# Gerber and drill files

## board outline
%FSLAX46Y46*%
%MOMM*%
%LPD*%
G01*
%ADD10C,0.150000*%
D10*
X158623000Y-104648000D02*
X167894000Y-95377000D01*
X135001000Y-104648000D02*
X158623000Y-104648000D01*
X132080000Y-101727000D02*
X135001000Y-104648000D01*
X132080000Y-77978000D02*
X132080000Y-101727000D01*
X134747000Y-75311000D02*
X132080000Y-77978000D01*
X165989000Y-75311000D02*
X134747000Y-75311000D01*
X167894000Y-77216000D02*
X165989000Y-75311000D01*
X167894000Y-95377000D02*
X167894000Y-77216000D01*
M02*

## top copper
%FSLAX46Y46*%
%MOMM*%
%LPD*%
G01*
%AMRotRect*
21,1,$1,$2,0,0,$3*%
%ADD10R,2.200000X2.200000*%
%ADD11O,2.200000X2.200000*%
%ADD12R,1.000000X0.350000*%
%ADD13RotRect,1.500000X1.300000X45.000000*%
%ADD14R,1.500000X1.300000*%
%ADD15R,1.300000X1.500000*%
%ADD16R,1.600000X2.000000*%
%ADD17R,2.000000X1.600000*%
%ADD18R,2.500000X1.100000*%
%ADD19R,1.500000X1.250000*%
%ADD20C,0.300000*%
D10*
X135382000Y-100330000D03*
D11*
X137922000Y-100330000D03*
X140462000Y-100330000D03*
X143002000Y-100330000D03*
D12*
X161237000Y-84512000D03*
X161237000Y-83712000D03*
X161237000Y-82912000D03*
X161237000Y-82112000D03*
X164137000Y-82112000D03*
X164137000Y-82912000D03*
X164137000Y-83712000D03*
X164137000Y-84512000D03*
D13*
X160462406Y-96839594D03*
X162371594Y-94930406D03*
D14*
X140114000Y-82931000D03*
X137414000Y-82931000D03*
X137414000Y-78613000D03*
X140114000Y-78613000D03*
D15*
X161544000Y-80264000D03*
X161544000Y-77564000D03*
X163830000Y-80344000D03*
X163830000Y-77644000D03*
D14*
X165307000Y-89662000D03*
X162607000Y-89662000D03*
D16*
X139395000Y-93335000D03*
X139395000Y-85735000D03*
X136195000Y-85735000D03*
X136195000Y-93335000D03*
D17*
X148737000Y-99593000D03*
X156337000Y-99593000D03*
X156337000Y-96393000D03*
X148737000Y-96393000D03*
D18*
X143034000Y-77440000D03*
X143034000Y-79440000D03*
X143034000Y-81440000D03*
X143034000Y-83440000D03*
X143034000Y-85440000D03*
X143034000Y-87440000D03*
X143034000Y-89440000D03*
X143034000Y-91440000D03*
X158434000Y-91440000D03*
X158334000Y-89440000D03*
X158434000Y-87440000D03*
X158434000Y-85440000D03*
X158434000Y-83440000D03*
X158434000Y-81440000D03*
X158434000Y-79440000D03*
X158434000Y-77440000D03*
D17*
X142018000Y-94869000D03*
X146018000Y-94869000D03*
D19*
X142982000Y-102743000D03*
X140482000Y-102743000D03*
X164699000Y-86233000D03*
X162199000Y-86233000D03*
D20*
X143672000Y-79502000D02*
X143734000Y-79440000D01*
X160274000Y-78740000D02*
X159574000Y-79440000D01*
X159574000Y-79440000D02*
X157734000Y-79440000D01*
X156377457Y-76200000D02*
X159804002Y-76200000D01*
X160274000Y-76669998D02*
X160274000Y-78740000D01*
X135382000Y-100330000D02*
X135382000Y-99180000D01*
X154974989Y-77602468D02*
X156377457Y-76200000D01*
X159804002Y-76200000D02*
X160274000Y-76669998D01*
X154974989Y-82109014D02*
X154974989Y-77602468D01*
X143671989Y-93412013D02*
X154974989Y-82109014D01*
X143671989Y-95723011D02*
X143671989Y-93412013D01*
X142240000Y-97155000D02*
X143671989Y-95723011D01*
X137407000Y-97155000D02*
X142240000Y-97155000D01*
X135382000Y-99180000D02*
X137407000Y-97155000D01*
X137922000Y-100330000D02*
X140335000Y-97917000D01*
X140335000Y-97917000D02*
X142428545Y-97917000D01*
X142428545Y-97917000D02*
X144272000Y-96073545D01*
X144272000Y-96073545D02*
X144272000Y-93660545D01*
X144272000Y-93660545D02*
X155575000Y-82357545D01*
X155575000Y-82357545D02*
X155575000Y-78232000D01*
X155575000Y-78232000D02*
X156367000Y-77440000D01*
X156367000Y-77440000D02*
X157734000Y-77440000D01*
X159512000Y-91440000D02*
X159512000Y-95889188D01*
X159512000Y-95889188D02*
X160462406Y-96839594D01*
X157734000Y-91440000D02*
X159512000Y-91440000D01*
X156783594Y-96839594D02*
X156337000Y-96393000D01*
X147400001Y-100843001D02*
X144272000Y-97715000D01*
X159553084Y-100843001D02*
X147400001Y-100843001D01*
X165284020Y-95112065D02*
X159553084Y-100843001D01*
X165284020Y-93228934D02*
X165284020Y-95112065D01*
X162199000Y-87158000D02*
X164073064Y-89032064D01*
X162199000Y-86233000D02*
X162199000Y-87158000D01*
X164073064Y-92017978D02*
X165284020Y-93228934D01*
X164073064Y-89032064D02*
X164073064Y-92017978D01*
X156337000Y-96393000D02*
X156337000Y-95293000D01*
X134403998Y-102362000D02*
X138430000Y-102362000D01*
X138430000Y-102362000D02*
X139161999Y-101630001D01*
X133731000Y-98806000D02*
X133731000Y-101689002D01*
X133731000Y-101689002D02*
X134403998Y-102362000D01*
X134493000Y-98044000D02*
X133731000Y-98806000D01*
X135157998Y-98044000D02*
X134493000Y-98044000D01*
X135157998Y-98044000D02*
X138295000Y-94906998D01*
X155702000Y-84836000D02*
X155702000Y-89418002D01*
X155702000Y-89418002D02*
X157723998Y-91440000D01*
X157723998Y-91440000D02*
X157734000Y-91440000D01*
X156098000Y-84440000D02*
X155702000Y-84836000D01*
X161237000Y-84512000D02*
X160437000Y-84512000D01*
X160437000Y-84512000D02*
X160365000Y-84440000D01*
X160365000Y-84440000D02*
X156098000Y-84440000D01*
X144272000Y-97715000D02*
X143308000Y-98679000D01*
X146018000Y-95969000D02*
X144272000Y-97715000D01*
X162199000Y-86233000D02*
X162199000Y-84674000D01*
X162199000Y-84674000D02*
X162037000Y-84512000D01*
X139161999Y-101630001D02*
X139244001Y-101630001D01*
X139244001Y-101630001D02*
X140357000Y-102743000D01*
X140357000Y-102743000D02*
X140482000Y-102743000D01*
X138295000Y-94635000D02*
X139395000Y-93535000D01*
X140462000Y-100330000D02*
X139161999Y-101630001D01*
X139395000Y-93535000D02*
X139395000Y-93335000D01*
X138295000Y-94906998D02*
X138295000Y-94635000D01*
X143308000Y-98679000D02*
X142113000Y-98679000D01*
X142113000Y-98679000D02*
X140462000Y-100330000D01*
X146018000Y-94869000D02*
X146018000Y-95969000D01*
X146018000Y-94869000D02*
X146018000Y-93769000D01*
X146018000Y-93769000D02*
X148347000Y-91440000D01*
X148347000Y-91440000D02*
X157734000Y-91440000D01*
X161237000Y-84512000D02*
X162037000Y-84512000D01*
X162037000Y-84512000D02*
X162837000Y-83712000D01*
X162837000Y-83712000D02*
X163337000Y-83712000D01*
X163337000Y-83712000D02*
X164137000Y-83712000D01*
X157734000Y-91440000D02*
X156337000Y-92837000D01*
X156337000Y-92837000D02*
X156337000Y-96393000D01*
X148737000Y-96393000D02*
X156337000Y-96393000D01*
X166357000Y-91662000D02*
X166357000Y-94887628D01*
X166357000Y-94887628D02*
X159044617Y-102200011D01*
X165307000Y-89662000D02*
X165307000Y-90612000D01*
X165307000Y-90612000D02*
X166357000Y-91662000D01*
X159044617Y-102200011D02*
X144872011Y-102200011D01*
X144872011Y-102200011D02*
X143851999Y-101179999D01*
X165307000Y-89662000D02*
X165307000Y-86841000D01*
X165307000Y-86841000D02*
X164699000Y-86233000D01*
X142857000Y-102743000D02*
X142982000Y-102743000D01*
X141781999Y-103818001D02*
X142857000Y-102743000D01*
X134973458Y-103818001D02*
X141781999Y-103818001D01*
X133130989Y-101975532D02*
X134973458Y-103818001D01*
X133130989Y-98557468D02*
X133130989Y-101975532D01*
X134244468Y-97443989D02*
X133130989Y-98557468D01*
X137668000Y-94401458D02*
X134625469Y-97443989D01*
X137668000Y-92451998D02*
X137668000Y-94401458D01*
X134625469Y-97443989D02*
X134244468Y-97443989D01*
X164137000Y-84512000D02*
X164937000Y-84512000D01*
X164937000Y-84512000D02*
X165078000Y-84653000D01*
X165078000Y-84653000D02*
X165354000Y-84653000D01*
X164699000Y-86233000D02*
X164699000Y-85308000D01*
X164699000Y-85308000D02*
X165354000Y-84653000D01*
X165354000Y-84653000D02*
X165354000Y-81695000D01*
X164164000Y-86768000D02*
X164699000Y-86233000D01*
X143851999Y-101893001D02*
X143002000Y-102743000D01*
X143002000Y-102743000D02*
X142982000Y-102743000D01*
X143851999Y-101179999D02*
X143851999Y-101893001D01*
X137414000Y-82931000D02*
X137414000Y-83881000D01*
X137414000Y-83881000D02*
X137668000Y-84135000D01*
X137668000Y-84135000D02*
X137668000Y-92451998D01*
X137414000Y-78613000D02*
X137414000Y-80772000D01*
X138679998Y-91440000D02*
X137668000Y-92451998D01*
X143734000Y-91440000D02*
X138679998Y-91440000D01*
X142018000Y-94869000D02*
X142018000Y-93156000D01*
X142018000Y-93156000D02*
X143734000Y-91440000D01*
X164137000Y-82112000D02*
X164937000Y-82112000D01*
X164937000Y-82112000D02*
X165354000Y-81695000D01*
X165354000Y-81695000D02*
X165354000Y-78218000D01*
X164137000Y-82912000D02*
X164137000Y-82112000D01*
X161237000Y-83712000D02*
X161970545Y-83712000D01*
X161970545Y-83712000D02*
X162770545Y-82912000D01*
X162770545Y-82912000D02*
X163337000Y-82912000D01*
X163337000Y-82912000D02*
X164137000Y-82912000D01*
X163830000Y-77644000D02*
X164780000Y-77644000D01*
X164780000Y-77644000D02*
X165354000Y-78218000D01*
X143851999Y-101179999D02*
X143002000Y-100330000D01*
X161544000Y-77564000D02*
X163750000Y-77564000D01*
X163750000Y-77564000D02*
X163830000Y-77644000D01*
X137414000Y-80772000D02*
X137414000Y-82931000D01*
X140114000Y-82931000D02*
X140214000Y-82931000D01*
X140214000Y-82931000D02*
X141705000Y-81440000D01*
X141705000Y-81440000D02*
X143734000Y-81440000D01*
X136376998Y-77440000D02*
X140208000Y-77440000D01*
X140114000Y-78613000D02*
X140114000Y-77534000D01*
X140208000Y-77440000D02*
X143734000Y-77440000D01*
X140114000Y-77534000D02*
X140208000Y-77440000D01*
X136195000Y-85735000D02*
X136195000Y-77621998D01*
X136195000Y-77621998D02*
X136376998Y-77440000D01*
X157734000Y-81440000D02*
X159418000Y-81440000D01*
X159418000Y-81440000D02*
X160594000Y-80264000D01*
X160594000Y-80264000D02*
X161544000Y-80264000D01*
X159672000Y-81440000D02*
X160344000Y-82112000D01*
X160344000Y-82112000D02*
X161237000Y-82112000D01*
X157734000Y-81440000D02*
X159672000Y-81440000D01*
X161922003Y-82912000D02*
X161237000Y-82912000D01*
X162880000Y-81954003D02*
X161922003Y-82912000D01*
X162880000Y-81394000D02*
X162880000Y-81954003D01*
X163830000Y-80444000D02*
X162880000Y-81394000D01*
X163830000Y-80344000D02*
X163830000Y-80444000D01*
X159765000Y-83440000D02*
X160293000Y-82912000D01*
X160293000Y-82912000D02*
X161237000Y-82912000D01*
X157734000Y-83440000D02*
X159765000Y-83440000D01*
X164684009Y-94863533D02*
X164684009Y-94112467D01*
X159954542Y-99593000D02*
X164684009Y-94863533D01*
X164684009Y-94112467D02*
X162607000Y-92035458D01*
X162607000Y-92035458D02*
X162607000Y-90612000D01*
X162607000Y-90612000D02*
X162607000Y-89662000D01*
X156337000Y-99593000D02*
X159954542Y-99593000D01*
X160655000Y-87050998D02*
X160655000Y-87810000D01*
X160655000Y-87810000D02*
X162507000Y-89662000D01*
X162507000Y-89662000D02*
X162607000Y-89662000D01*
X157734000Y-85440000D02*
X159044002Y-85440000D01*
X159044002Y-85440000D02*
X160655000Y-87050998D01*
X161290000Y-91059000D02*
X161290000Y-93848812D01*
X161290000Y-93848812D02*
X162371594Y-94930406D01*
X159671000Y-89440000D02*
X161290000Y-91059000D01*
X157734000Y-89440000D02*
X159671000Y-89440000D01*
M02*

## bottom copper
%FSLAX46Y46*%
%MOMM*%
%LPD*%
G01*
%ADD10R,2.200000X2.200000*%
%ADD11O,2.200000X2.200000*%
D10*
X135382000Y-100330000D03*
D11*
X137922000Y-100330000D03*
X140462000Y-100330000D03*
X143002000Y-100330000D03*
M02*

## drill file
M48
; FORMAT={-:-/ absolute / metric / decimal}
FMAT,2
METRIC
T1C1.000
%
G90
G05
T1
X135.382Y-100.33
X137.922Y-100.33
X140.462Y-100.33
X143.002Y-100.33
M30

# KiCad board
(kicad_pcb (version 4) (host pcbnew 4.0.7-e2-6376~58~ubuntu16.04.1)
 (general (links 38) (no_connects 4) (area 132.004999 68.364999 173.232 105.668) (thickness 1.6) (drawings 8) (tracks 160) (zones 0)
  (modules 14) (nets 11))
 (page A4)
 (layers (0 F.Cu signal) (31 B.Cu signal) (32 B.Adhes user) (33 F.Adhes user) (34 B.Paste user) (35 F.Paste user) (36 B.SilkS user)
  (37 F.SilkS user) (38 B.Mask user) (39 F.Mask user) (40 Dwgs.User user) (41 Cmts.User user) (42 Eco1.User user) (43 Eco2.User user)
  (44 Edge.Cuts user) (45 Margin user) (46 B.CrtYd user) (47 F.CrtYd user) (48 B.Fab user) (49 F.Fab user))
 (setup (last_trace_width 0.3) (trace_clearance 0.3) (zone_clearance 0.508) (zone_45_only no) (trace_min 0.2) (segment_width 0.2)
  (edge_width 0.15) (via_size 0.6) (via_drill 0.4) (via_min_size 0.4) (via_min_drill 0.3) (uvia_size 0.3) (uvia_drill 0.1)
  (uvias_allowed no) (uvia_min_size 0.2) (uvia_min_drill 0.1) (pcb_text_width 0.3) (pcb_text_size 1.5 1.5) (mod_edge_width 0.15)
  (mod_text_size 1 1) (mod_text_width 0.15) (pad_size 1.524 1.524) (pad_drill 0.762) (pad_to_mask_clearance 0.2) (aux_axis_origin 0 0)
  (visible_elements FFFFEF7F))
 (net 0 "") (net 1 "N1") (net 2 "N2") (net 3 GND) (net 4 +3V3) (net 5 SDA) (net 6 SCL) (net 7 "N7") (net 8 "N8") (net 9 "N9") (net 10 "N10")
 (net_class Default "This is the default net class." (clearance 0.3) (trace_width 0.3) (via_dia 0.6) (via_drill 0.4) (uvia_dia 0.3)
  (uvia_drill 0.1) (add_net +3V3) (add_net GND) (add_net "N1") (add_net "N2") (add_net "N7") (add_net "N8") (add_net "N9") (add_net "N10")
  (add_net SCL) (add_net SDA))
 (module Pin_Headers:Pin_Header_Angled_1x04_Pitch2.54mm (layer F.Cu) (at 135.382 100.33 90)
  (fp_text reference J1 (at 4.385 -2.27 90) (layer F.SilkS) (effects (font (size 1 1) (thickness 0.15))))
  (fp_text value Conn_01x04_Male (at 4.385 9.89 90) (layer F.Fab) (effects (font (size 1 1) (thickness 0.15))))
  (pad 1 thru_hole rect (at 0 0 90) (size 2.2 2.2) (drill 1) (layers *.Cu *.Mask) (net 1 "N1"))
  (pad 2 thru_hole oval (at 0 2.54 90) (size 2.2 2.2) (drill 1) (layers *.Cu *.Mask) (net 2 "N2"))
  (pad 3 thru_hole oval (at 0 5.08 90) (size 2.2 2.2) (drill 1) (layers *.Cu *.Mask) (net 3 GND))
  (pad 4 thru_hole oval (at 0 7.62 90) (size 2.2 2.2) (drill 1) (layers *.Cu *.Mask) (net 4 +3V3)))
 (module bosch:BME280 (layer F.Cu) (at 162.687 83.312 180)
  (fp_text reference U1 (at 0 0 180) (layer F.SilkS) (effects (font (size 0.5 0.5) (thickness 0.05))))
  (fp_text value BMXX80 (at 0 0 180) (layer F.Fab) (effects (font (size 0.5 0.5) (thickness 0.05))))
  (pad 1 smd rect (at 1.45 -1.2 180) (size 1 0.35) (layers F.Cu F.Paste F.Mask) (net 3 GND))
  (pad 2 smd rect (at 1.45 -0.4 180) (size 1 0.35) (layers F.Cu F.Paste F.Mask) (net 4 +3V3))
  (pad 3 smd rect (at 1.45 0.4 180) (size 1 0.35) (layers F.Cu F.Paste F.Mask) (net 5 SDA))
  (pad 4 smd rect (at 1.45 1.2 180) (size 1 0.35) (layers F.Cu F.Paste F.Mask) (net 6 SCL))
  (pad 5 smd rect (at -1.45 1.2 180) (size 1 0.35) (layers F.Cu F.Paste F.Mask) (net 4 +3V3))
  (pad 6 smd rect (at -1.45 0.4 180) (size 1 0.35) (layers F.Cu F.Paste F.Mask) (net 4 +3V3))
  (pad 7 smd rect (at -1.45 -0.4 180) (size 1 0.35) (layers F.Cu F.Paste F.Mask) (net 3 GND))
  (pad 8 smd rect (at -1.45 -1.2 180) (size 1 0.35) (layers F.Cu F.Paste F.Mask) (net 4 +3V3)))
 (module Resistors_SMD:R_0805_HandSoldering (layer F.Cu) (at 161.417 95.885 45)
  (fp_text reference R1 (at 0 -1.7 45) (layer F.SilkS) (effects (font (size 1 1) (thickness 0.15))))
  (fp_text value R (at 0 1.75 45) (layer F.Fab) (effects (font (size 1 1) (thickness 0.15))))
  (pad 1 smd rect (at -1.35 0 45) (size 1.5 1.3) (layers F.Cu F.Paste F.Mask) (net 3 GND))
  (pad 2 smd rect (at 1.35 0 45) (size 1.5 1.3) (layers F.Cu F.Paste F.Mask) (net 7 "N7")))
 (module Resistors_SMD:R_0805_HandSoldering (layer F.Cu) (at 138.764 82.931 180)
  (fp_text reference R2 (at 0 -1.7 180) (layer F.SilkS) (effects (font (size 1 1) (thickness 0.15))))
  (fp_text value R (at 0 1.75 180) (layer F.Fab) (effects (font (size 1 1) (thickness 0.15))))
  (pad 1 smd rect (at -1.35 0 180) (size 1.5 1.3) (layers F.Cu F.Paste F.Mask) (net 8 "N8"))
  (pad 2 smd rect (at 1.35 0 180) (size 1.5 1.3) (layers F.Cu F.Paste F.Mask) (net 4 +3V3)))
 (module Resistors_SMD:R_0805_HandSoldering (layer F.Cu) (at 138.764 78.613)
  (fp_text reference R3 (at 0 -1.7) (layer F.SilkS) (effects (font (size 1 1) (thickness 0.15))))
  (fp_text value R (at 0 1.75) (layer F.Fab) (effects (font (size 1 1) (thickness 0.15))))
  (pad 1 smd rect (at -1.35 0) (size 1.5 1.3) (layers F.Cu F.Paste F.Mask) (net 4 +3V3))
  (pad 2 smd rect (at 1.35 0) (size 1.5 1.3) (layers F.Cu F.Paste F.Mask) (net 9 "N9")))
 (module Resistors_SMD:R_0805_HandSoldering (layer F.Cu) (at 161.544 78.914 90)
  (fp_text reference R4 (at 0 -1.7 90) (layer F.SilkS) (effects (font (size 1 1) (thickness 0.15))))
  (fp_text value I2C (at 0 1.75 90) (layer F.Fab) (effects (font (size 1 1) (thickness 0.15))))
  (pad 1 smd rect (at -1.35 0 90) (size 1.5 1.3) (layers F.Cu F.Paste F.Mask) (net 6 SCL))
  (pad 2 smd rect (at 1.35 0 90) (size 1.5 1.3) (layers F.Cu F.Paste F.Mask) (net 4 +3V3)))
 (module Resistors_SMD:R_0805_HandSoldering (layer F.Cu) (at 163.83 78.994 90)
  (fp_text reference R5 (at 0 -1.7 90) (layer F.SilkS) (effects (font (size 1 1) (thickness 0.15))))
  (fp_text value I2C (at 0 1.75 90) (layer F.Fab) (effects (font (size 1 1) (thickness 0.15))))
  (pad 1 smd rect (at -1.35 0 90) (size 1.5 1.3) (layers F.Cu F.Paste F.Mask) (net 5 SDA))
  (pad 2 smd rect (at 1.35 0 90) (size 1.5 1.3) (layers F.Cu F.Paste F.Mask) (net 4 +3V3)))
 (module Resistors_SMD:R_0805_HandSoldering (layer F.Cu) (at 163.957 89.662 180)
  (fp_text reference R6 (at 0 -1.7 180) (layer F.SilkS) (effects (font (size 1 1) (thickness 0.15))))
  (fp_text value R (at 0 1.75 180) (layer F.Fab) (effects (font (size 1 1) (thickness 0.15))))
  (pad 1 smd rect (at -1.35 0 180) (size 1.5 1.3) (layers F.Cu F.Paste F.Mask) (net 4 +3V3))
  (pad 2 smd rect (at 1.35 0 180) (size 1.5 1.3) (layers F.Cu F.Paste F.Mask) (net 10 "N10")))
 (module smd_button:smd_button (layer F.Cu) (at 137.795 89.535 270)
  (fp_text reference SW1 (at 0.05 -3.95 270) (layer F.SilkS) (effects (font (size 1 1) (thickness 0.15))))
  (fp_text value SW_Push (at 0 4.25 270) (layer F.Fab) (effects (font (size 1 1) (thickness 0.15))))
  (pad 1 smd rect (at 3.8 -1.6 270) (size 2 1.6) (layers F.Cu F.Paste F.Mask) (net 3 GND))
  (pad 1 smd rect (at -3.8 -1.6 270) (size 2 1.6) (layers F.Cu F.Paste F.Mask) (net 3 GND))
  (pad 2 smd rect (at -3.8 1.6 270) (size 2 1.6) (layers F.Cu F.Paste F.Mask) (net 9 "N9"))
  (pad 2 smd rect (at 3.8 1.6 270) (size 2 1.6) (layers F.Cu F.Paste F.Mask) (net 9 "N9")))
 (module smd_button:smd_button (layer F.Cu) (at 152.537 97.993 180)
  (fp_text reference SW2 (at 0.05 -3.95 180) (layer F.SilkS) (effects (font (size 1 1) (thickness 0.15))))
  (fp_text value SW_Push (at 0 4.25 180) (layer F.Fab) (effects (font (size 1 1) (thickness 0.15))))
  (pad 1 smd rect (at 3.8 -1.6 180) (size 2 1.6) (layers F.Cu F.Paste F.Mask) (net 10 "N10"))
  (pad 1 smd rect (at -3.8 -1.6 180) (size 2 1.6) (layers F.Cu F.Paste F.Mask) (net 10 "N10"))
  (pad 2 smd rect (at -3.8 1.6 180) (size 2 1.6) (layers F.Cu F.Paste F.Mask) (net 3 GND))
  (pad 2 smd rect (at 3.8 1.6 180) (size 2 1.6) (layers F.Cu F.Paste F.Mask) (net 3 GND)))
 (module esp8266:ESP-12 (layer F.Cu) (at 143.734 77.44)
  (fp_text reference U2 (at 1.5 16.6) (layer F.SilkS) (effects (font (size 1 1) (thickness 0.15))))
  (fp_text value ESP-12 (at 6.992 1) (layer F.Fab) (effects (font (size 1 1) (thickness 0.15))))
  (pad 1 smd rect (at 0 0) (size 2.5 1.1) (drill (offset -0.7 0)) (layers F.Cu F.Paste F.Mask) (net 9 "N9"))
  (pad 2 smd rect (at 0 2) (size 2.5 1.1) (drill (offset -0.7 0)) (layers F.Cu F.Paste F.Mask))
  (pad 3 smd rect (at 0 4) (size 2.5 1.1) (drill (offset -0.7 0)) (layers F.Cu F.Paste F.Mask) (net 8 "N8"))
  (pad 4 smd rect (at 0 6) (size 2.5 1.1) (drill (offset -0.7 0)) (layers F.Cu F.Paste F.Mask))
  (pad 5 smd rect (at 0 8) (size 2.5 1.1) (drill (offset -0.7 0)) (layers F.Cu F.Paste F.Mask))
  (pad 6 smd rect (at 0 10) (size 2.5 1.1) (drill (offset -0.7 0)) (layers F.Cu F.Paste F.Mask))
  (pad 7 smd rect (at 0 12) (size 2.5 1.1) (drill (offset -0.7 0)) (layers F.Cu F.Paste F.Mask))
  (pad 8 smd rect (at 0 14) (size 2.5 1.1) (drill (offset -0.7 0)) (layers F.Cu F.Paste F.Mask) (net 4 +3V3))
  (pad 9 smd rect (at 14 14) (size 2.5 1.1) (drill (offset 0.7 0)) (layers F.Cu F.Paste F.Mask) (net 3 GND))
  (pad 10 smd rect (at 14 12) (size 2.5 1.1) (drill (offset 0.6 0)) (layers F.Cu F.Paste F.Mask) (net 7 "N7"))
  (pad 11 smd rect (at 14 10) (size 2.5 1.1) (drill (offset 0.7 0)) (layers F.Cu F.Paste F.Mask))
  (pad 12 smd rect (at 14 8) (size 2.5 1.1) (drill (offset 0.7 0)) (layers F.Cu F.Paste F.Mask) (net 10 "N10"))
  (pad 13 smd rect (at 14 6) (size 2.5 1.1) (drill (offset 0.7 0)) (layers F.Cu F.Paste F.Mask) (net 5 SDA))
  (pad 14 smd rect (at 14 4) (size 2.5 1.1) (drill (offset 0.7 0)) (layers F.Cu F.Paste F.Mask) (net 6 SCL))
  (pad 15 smd rect (at 14 2) (size 2.5 1.1) (drill (offset 0.7 0)) (layers F.Cu F.Paste F.Mask) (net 1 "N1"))
  (pad 16 smd rect (at 14 0) (size 2.5 1.1) (drill (offset 0.7 0)) (layers F.Cu F.Paste F.Mask) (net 2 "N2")))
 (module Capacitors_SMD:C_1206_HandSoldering (layer F.Cu) (at 144.018 94.869)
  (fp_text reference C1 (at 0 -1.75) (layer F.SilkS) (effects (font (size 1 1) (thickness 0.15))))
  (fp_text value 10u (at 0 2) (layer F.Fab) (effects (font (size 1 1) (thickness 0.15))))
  (pad 1 smd rect (at -2 0) (size 2 1.6) (layers F.Cu F.Paste F.Mask) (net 4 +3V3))
  (pad 2 smd rect (at 2 0) (size 2 1.6) (layers F.Cu F.Paste F.Mask) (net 3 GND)))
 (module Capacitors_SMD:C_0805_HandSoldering (layer F.Cu) (at 141.732 102.743 180)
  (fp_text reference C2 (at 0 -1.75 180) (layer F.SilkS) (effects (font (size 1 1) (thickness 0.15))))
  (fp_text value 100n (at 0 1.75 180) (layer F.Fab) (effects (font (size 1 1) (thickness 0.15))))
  (pad 1 smd rect (at -1.25 0 180) (size 1.5 1.25) (layers F.Cu F.Paste F.Mask) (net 4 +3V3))
  (pad 2 smd rect (at 1.25 0 180) (size 1.5 1.25) (layers F.Cu F.Paste F.Mask) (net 3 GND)))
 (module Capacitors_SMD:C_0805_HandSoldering (layer F.Cu) (at 163.449 86.233 180)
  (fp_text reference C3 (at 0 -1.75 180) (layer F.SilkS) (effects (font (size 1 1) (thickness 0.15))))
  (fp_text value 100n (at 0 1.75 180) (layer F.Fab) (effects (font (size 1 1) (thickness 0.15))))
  (pad 1 smd rect (at -1.25 0 180) (size 1.5 1.25) (layers F.Cu F.Paste F.Mask) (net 4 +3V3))
  (pad 2 smd rect (at 1.25 0 180) (size 1.5 1.25) (layers F.Cu F.Paste F.Mask) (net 3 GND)))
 (gr_line (start 158.623 104.648) (end 167.894 95.377) (layer Edge.Cuts) (width 0.15))
 (gr_line (start 135.001 104.648) (end 158.623 104.648) (layer Edge.Cuts) (width 0.15))
 (gr_line (start 132.08 101.727) (end 135.001 104.648) (layer Edge.Cuts) (width 0.15))
 (gr_line (start 132.08 77.978) (end 132.08 101.727) (layer Edge.Cuts) (width 0.15))
 (gr_line (start 134.747 75.311) (end 132.08 77.978) (layer Edge.Cuts) (width 0.15))
 (gr_line (start 165.989 75.311) (end 134.747 75.311) (layer Edge.Cuts) (width 0.15))
 (gr_line (start 167.894 77.216) (end 165.989 75.311) (layer Edge.Cuts) (width 0.15))
 (gr_line (start 167.894 95.377) (end 167.894 77.216) (layer Edge.Cuts) (width 0.15))
 (segment (start 143.672 79.502) (end 143.734 79.44) (width 0.3) (layer F.Cu) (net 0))
 (segment (start 160.274 78.74) (end 159.574 79.44) (width 0.3) (layer F.Cu) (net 1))
 (segment (start 159.574 79.44) (end 157.734 79.44) (width 0.3) (layer F.Cu) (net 1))
 (segment (start 156.377457 76.2) (end 159.804002 76.2) (width 0.3) (layer F.Cu) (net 1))
 (segment (start 160.274 76.669998) (end 160.274 78.74) (width 0.3) (layer F.Cu) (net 1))
 (segment (start 135.382 100.33) (end 135.382 99.18) (width 0.3) (layer F.Cu) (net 1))
 (segment (start 154.974989 77.602468) (end 156.377457 76.2) (width 0.3) (layer F.Cu) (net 1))
 (segment (start 159.804002 76.2) (end 160.274 76.669998) (width 0.3) (layer F.Cu) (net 1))
 (segment (start 154.974989 82.109014) (end 154.974989 77.602468) (width 0.3) (layer F.Cu) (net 1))
 (segment (start 143.671989 93.412013) (end 154.974989 82.109014) (width 0.3) (layer F.Cu) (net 1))
 (segment (start 143.671989 95.723011) (end 143.671989 93.412013) (width 0.3) (layer F.Cu) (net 1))
 (segment (start 142.24 97.155) (end 143.671989 95.723011) (width 0.3) (layer F.Cu) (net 1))
 (segment (start 137.407 97.155) (end 142.24 97.155) (width 0.3) (layer F.Cu) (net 1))
 (segment (start 135.382 99.18) (end 137.407 97.155) (width 0.3) (layer F.Cu) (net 1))
 (segment (start 137.922 100.33) (end 140.335 97.917) (width 0.3) (layer F.Cu) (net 2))
 (segment (start 140.335 97.917) (end 142.428545 97.917) (width 0.3) (layer F.Cu) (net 2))
 (segment (start 142.428545 97.917) (end 144.272 96.073545) (width 0.3) (layer F.Cu) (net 2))
 (segment (start 144.272 96.073545) (end 144.272 93.660545) (width 0.3) (layer F.Cu) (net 2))
 (segment (start 144.272 93.660545) (end 155.575 82.357545) (width 0.3) (layer F.Cu) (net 2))
 (segment (start 155.575 82.357545) (end 155.575 78.232) (width 0.3) (layer F.Cu) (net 2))
 (segment (start 155.575 78.232) (end 156.367 77.44) (width 0.3) (layer F.Cu) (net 2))
 (segment (start 156.367 77.44) (end 157.734 77.44) (width 0.3) (layer F.Cu) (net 2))
 (segment (start 159.512 91.44) (end 159.512 95.889188) (width 0.3) (layer F.Cu) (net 3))
 (segment (start 159.512 95.889188) (end 160.462406 96.839594) (width 0.3) (layer F.Cu) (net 3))
 (segment (start 157.734 91.44) (end 159.512 91.44) (width 0.3) (layer F.Cu) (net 3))
 (segment (start 156.783594 96.839594) (end 156.337 96.393) (width 0.3) (layer F.Cu) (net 3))
 (segment (start 147.400001 100.843001) (end 144.272 97.715) (width 0.3) (layer F.Cu) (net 3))
 (segment (start 159.553084 100.843001) (end 147.400001 100.843001) (width 0.3) (layer F.Cu) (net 3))
 (segment (start 165.28402 95.112065) (end 159.553084 100.843001) (width 0.3) (layer F.Cu) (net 3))
 (segment (start 165.28402 93.228934) (end 165.28402 95.112065) (width 0.3) (layer F.Cu) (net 3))
 (segment (start 162.199 87.158) (end 164.073064 89.032064) (width 0.3) (layer F.Cu) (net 3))
 (segment (start 162.199 86.233) (end 162.199 87.158) (width 0.3) (layer F.Cu) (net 3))
 (segment (start 164.073064 92.017978) (end 165.28402 93.228934) (width 0.3) (layer F.Cu) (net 3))
 (segment (start 164.073064 89.032064) (end 164.073064 92.017978) (width 0.3) (layer F.Cu) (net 3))
 (segment (start 156.337 96.393) (end 156.337 95.293) (width 0.3) (layer F.Cu) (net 3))
 (segment (start 134.403998 102.362) (end 138.43 102.362) (width 0.3) (layer F.Cu) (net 3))
 (segment (start 138.43 102.362) (end 139.161999 101.630001) (width 0.3) (layer F.Cu) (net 3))
 (segment (start 133.731 98.806) (end 133.731 101.689002) (width 0.3) (layer F.Cu) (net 3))
 (segment (start 133.731 101.689002) (end 134.403998 102.362) (width 0.3) (layer F.Cu) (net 3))
 (segment (start 134.493 98.044) (end 133.731 98.806) (width 0.3) (layer F.Cu) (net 3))
 (segment (start 135.157998 98.044) (end 134.493 98.044) (width 0.3) (layer F.Cu) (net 3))
 (segment (start 135.157998 98.044) (end 138.295 94.906998) (width 0.3) (layer F.Cu) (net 3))
 (segment (start 155.702 84.836) (end 155.702 89.418002) (width 0.3) (layer F.Cu) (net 3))
 (segment (start 155.702 89.418002) (end 157.723998 91.44) (width 0.3) (layer F.Cu) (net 3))
 (segment (start 157.723998 91.44) (end 157.734 91.44) (width 0.3) (layer F.Cu) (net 3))
 (segment (start 156.098 84.44) (end 155.702 84.836) (width 0.3) (layer F.Cu) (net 3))
 (segment (start 161.237 84.512) (end 160.437 84.512) (width 0.3) (layer F.Cu) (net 3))
 (segment (start 160.437 84.512) (end 160.365 84.44) (width 0.3) (layer F.Cu) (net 3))
 (segment (start 160.365 84.44) (end 156.098 84.44) (width 0.3) (layer F.Cu) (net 3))
 (segment (start 144.272 97.715) (end 143.308 98.679) (width 0.3) (layer F.Cu) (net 3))
 (segment (start 146.018 95.969) (end 144.272 97.715) (width 0.3) (layer F.Cu) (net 3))
 (segment (start 162.199 86.233) (end 162.199 84.674) (width 0.3) (layer F.Cu) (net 3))
 (segment (start 162.199 84.674) (end 162.037 84.512) (width 0.3) (layer F.Cu) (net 3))
 (segment (start 139.161999 101.630001) (end 139.244001 101.630001) (width 0.3) (layer F.Cu) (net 3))
 (segment (start 139.244001 101.630001) (end 140.357 102.743) (width 0.3) (layer F.Cu) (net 3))
 (segment (start 140.357 102.743) (end 140.482 102.743) (width 0.3) (layer F.Cu) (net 3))
 (segment (start 138.295 94.635) (end 139.395 93.535) (width 0.3) (layer F.Cu) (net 3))
 (segment (start 140.462 100.33) (end 139.161999 101.630001) (width 0.3) (layer F.Cu) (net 3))
 (segment (start 139.395 93.535) (end 139.395 93.335) (width 0.3) (layer F.Cu) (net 3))
 (segment (start 138.295 94.906998) (end 138.295 94.635) (width 0.3) (layer F.Cu) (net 3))
 (segment (start 143.308 98.679) (end 142.113 98.679) (width 0.3) (layer F.Cu) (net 3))
 (segment (start 142.113 98.679) (end 140.462 100.33) (width 0.3) (layer F.Cu) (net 3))
 (segment (start 146.018 94.869) (end 146.018 95.969) (width 0.3) (layer F.Cu) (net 3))
 (segment (start 146.018 94.869) (end 146.018 93.769) (width 0.3) (layer F.Cu) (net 3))
 (segment (start 146.018 93.769) (end 148.347 91.44) (width 0.3) (layer F.Cu) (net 3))
 (segment (start 148.347 91.44) (end 157.734 91.44) (width 0.3) (layer F.Cu) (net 3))
 (segment (start 161.237 84.512) (end 162.037 84.512) (width 0.3) (layer F.Cu) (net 3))
 (segment (start 162.037 84.512) (end 162.837 83.712) (width 0.3) (layer F.Cu) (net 3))
 (segment (start 162.837 83.712) (end 163.337 83.712) (width 0.3) (layer F.Cu) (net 3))
 (segment (start 163.337 83.712) (end 164.137 83.712) (width 0.3) (layer F.Cu) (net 3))
 (segment (start 157.734 91.44) (end 156.337 92.837) (width 0.3) (layer F.Cu) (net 3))
 (segment (start 156.337 92.837) (end 156.337 96.393) (width 0.3) (layer F.Cu) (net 3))
 (segment (start 148.737 96.393) (end 156.337 96.393) (width 0.3) (layer F.Cu) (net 3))
 (segment (start 166.357 91.662) (end 166.357 94.887628) (width 0.3) (layer F.Cu) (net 4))
 (segment (start 166.357 94.887628) (end 159.044617 102.200011) (width 0.3) (layer F.Cu) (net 4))
 (segment (start 165.307 89.662) (end 165.307 90.612) (width 0.3) (layer F.Cu) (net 4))
 (segment (start 165.307 90.612) (end 166.357 91.662) (width 0.3) (layer F.Cu) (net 4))
 (segment (start 159.044617 102.200011) (end 144.872011 102.200011) (width 0.3) (layer F.Cu) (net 4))
 (segment (start 144.872011 102.200011) (end 143.851999 101.179999) (width 0.3) (layer F.Cu) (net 4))
 (segment (start 165.307 89.662) (end 165.307 86.841) (width 0.3) (layer F.Cu) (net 4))
 (segment (start 165.307 86.841) (end 164.699 86.233) (width 0.3) (layer F.Cu) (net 4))
 (segment (start 142.857 102.743) (end 142.982 102.743) (width 0.3) (layer F.Cu) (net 4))
 (segment (start 141.781999 103.818001) (end 142.857 102.743) (width 0.3) (layer F.Cu) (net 4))
 (segment (start 134.973458 103.818001) (end 141.781999 103.818001) (width 0.3) (layer F.Cu) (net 4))
 (segment (start 133.130989 101.975532) (end 134.973458 103.818001) (width 0.3) (layer F.Cu) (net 4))
 (segment (start 133.130989 98.557468) (end 133.130989 101.975532) (width 0.3) (layer F.Cu) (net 4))
 (segment (start 134.244468 97.443989) (end 133.130989 98.557468) (width 0.3) (layer F.Cu) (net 4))
 (segment (start 137.668 94.401458) (end 134.625469 97.443989) (width 0.3) (layer F.Cu) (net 4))
 (segment (start 137.668 92.451998) (end 137.668 94.401458) (width 0.3) (layer F.Cu) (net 4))
 (segment (start 134.625469 97.443989) (end 134.244468 97.443989) (width 0.3) (layer F.Cu) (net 4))
 (segment (start 164.137 84.512) (end 164.937 84.512) (width 0.3) (layer F.Cu) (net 4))
 (segment (start 164.937 84.512) (end 165.078 84.653) (width 0.3) (layer F.Cu) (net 4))
 (segment (start 165.078 84.653) (end 165.354 84.653) (width 0.3) (layer F.Cu) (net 4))
 (segment (start 164.699 86.233) (end 164.699 85.308) (width 0.3) (layer F.Cu) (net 4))
 (segment (start 164.699 85.308) (end 165.354 84.653) (width 0.3) (layer F.Cu) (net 4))
 (segment (start 165.354 84.653) (end 165.354 81.695) (width 0.3) (layer F.Cu) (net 4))
 (segment (start 164.164 86.768) (end 164.699 86.233) (width 0.3) (layer F.Cu) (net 4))
 (segment (start 143.851999 101.893001) (end 143.002 102.743) (width 0.3) (layer F.Cu) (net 4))
 (segment (start 143.002 102.743) (end 142.982 102.743) (width 0.3) (layer F.Cu) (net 4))
 (segment (start 143.851999 101.179999) (end 143.851999 101.893001) (width 0.3) (layer F.Cu) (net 4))
 (segment (start 137.414 82.931) (end 137.414 83.881) (width 0.3) (layer F.Cu) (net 4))
 (segment (start 137.414 83.881) (end 137.668 84.135) (width 0.3) (layer F.Cu) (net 4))
 (segment (start 137.668 84.135) (end 137.668 92.451998) (width 0.3) (layer F.Cu) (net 4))
 (segment (start 137.414 78.613) (end 137.414 80.772) (width 0.3) (layer F.Cu) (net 4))
 (segment (start 138.679998 91.44) (end 137.668 92.451998) (width 0.3) (layer F.Cu) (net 4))
 (segment (start 143.734 91.44) (end 138.679998 91.44) (width 0.3) (layer F.Cu) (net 4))
 (segment (start 142.018 94.869) (end 142.018 93.156) (width 0.3) (layer F.Cu) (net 4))
 (segment (start 142.018 93.156) (end 143.734 91.44) (width 0.3) (layer F.Cu) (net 4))
 (segment (start 164.137 82.112) (end 164.937 82.112) (width 0.3) (layer F.Cu) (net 4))
 (segment (start 164.937 82.112) (end 165.354 81.695) (width 0.3) (layer F.Cu) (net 4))
 (segment (start 165.354 81.695) (end 165.354 78.218) (width 0.3) (layer F.Cu) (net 4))
 (segment (start 164.137 82.912) (end 164.137 82.112) (width 0.3) (layer F.Cu) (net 4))
 (segment (start 161.237 83.712) (end 161.970545 83.712) (width 0.3) (layer F.Cu) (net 4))
 (segment (start 161.970545 83.712) (end 162.770545 82.912) (width 0.3) (layer F.Cu) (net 4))
 (segment (start 162.770545 82.912) (end 163.337 82.912) (width 0.3) (layer F.Cu) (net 4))
 (segment (start 163.337 82.912) (end 164.137 82.912) (width 0.3) (layer F.Cu) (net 4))
 (segment (start 163.83 77.644) (end 164.78 77.644) (width 0.3) (layer F.Cu) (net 4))
 (segment (start 164.78 77.644) (end 165.354 78.218) (width 0.3) (layer F.Cu) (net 4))
 (segment (start 143.851999 101.179999) (end 143.002 100.33) (width 0.3) (layer F.Cu) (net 4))
 (segment (start 161.544 77.564) (end 163.75 77.564) (width 0.3) (layer F.Cu) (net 4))
 (segment (start 163.75 77.564) (end 163.83 77.644) (width 0.3) (layer F.Cu) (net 4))
 (segment (start 137.414 80.772) (end 137.414 82.931) (width 0.3) (layer F.Cu) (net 4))
 (segment (start 140.114 82.931) (end 140.214 82.931) (width 0.3) (layer F.Cu) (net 8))
 (segment (start 140.214 82.931) (end 141.705 81.44) (width 0.3) (layer F.Cu) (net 8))
 (segment (start 141.705 81.44) (end 143.734 81.44) (width 0.3) (layer F.Cu) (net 8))
 (segment (start 136.376998 77.44) (end 140.208 77.44) (width 0.3) (layer F.Cu) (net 9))
 (segment (start 140.114 78.613) (end 140.114 77.534) (width 0.3) (layer F.Cu) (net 9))
 (segment (start 140.208 77.44) (end 143.734 77.44) (width 0.3) (layer F.Cu) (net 9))
 (segment (start 140.114 77.534) (end 140.208 77.44) (width 0.3) (layer F.Cu) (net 9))
 (segment (start 136.195 85.735) (end 136.195 77.621998) (width 0.3) (layer F.Cu) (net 9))
 (segment (start 136.195 77.621998) (end 136.376998 77.44) (width 0.3) (layer F.Cu) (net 9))
 (segment (start 157.734 81.44) (end 159.418 81.44) (width 0.3) (layer F.Cu) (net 6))
 (segment (start 159.418 81.44) (end 160.594 80.264) (width 0.3) (layer F.Cu) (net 6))
 (segment (start 160.594 80.264) (end 161.544 80.264) (width 0.3) (layer F.Cu) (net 6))
 (segment (start 159.672 81.44) (end 160.344 82.112) (width 0.3) (layer F.Cu) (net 6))
 (segment (start 160.344 82.112) (end 161.237 82.112) (width 0.3) (layer F.Cu) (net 6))
 (segment (start 157.734 81.44) (end 159.672 81.44) (width 0.3) (layer F.Cu) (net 6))
 (segment (start 161.922003 82.912) (end 161.237 82.912) (width 0.3) (layer F.Cu) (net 5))
 (segment (start 162.88 81.954003) (end 161.922003 82.912) (width 0.3) (layer F.Cu) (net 5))
 (segment (start 162.88 81.394) (end 162.88 81.954003) (width 0.3) (layer F.Cu) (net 5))
 (segment (start 163.83 80.444) (end 162.88 81.394) (width 0.3) (layer F.Cu) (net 5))
 (segment (start 163.83 80.344) (end 163.83 80.444) (width 0.3) (layer F.Cu) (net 5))
 (segment (start 159.765 83.44) (end 160.293 82.912) (width 0.3) (layer F.Cu) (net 5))
 (segment (start 160.293 82.912) (end 161.237 82.912) (width 0.3) (layer F.Cu) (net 5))
 (segment (start 157.734 83.44) (end 159.765 83.44) (width 0.3) (layer F.Cu) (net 5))
 (segment (start 164.684009 94.863533) (end 164.684009 94.112467) (width 0.3) (layer F.Cu) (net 10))
 (segment (start 159.954542 99.593) (end 164.684009 94.863533) (width 0.3) (layer F.Cu) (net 10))
 (segment (start 164.684009 94.112467) (end 162.607 92.035458) (width 0.3) (layer F.Cu) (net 10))
 (segment (start 162.607 92.035458) (end 162.607 90.612) (width 0.3) (layer F.Cu) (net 10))
 (segment (start 162.607 90.612) (end 162.607 89.662) (width 0.3) (layer F.Cu) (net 10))
 (segment (start 156.337 99.593) (end 159.954542 99.593) (width 0.3) (layer F.Cu) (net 10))
 (segment (start 160.655 87.050998) (end 160.655 87.81) (width 0.3) (layer F.Cu) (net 10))
 (segment (start 160.655 87.81) (end 162.507 89.662) (width 0.3) (layer F.Cu) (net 10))
 (segment (start 162.507 89.662) (end 162.607 89.662) (width 0.3) (layer F.Cu) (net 10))
 (segment (start 157.734 85.44) (end 159.044002 85.44) (width 0.3) (layer F.Cu) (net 10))
 (segment (start 159.044002 85.44) (end 160.655 87.050998) (width 0.3) (layer F.Cu) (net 10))
 (segment (start 161.29 91.059) (end 161.29 93.848812) (width 0.3) (layer F.Cu) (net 7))
 (segment (start 161.29 93.848812) (end 162.371594 94.930406) (width 0.3) (layer F.Cu) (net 7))
 (segment (start 159.671 89.44) (end 161.29 91.059) (width 0.3) (layer F.Cu) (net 7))
 (segment (start 157.734 89.44) (end 159.671 89.44) (width 0.3) (layer F.Cu) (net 7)))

